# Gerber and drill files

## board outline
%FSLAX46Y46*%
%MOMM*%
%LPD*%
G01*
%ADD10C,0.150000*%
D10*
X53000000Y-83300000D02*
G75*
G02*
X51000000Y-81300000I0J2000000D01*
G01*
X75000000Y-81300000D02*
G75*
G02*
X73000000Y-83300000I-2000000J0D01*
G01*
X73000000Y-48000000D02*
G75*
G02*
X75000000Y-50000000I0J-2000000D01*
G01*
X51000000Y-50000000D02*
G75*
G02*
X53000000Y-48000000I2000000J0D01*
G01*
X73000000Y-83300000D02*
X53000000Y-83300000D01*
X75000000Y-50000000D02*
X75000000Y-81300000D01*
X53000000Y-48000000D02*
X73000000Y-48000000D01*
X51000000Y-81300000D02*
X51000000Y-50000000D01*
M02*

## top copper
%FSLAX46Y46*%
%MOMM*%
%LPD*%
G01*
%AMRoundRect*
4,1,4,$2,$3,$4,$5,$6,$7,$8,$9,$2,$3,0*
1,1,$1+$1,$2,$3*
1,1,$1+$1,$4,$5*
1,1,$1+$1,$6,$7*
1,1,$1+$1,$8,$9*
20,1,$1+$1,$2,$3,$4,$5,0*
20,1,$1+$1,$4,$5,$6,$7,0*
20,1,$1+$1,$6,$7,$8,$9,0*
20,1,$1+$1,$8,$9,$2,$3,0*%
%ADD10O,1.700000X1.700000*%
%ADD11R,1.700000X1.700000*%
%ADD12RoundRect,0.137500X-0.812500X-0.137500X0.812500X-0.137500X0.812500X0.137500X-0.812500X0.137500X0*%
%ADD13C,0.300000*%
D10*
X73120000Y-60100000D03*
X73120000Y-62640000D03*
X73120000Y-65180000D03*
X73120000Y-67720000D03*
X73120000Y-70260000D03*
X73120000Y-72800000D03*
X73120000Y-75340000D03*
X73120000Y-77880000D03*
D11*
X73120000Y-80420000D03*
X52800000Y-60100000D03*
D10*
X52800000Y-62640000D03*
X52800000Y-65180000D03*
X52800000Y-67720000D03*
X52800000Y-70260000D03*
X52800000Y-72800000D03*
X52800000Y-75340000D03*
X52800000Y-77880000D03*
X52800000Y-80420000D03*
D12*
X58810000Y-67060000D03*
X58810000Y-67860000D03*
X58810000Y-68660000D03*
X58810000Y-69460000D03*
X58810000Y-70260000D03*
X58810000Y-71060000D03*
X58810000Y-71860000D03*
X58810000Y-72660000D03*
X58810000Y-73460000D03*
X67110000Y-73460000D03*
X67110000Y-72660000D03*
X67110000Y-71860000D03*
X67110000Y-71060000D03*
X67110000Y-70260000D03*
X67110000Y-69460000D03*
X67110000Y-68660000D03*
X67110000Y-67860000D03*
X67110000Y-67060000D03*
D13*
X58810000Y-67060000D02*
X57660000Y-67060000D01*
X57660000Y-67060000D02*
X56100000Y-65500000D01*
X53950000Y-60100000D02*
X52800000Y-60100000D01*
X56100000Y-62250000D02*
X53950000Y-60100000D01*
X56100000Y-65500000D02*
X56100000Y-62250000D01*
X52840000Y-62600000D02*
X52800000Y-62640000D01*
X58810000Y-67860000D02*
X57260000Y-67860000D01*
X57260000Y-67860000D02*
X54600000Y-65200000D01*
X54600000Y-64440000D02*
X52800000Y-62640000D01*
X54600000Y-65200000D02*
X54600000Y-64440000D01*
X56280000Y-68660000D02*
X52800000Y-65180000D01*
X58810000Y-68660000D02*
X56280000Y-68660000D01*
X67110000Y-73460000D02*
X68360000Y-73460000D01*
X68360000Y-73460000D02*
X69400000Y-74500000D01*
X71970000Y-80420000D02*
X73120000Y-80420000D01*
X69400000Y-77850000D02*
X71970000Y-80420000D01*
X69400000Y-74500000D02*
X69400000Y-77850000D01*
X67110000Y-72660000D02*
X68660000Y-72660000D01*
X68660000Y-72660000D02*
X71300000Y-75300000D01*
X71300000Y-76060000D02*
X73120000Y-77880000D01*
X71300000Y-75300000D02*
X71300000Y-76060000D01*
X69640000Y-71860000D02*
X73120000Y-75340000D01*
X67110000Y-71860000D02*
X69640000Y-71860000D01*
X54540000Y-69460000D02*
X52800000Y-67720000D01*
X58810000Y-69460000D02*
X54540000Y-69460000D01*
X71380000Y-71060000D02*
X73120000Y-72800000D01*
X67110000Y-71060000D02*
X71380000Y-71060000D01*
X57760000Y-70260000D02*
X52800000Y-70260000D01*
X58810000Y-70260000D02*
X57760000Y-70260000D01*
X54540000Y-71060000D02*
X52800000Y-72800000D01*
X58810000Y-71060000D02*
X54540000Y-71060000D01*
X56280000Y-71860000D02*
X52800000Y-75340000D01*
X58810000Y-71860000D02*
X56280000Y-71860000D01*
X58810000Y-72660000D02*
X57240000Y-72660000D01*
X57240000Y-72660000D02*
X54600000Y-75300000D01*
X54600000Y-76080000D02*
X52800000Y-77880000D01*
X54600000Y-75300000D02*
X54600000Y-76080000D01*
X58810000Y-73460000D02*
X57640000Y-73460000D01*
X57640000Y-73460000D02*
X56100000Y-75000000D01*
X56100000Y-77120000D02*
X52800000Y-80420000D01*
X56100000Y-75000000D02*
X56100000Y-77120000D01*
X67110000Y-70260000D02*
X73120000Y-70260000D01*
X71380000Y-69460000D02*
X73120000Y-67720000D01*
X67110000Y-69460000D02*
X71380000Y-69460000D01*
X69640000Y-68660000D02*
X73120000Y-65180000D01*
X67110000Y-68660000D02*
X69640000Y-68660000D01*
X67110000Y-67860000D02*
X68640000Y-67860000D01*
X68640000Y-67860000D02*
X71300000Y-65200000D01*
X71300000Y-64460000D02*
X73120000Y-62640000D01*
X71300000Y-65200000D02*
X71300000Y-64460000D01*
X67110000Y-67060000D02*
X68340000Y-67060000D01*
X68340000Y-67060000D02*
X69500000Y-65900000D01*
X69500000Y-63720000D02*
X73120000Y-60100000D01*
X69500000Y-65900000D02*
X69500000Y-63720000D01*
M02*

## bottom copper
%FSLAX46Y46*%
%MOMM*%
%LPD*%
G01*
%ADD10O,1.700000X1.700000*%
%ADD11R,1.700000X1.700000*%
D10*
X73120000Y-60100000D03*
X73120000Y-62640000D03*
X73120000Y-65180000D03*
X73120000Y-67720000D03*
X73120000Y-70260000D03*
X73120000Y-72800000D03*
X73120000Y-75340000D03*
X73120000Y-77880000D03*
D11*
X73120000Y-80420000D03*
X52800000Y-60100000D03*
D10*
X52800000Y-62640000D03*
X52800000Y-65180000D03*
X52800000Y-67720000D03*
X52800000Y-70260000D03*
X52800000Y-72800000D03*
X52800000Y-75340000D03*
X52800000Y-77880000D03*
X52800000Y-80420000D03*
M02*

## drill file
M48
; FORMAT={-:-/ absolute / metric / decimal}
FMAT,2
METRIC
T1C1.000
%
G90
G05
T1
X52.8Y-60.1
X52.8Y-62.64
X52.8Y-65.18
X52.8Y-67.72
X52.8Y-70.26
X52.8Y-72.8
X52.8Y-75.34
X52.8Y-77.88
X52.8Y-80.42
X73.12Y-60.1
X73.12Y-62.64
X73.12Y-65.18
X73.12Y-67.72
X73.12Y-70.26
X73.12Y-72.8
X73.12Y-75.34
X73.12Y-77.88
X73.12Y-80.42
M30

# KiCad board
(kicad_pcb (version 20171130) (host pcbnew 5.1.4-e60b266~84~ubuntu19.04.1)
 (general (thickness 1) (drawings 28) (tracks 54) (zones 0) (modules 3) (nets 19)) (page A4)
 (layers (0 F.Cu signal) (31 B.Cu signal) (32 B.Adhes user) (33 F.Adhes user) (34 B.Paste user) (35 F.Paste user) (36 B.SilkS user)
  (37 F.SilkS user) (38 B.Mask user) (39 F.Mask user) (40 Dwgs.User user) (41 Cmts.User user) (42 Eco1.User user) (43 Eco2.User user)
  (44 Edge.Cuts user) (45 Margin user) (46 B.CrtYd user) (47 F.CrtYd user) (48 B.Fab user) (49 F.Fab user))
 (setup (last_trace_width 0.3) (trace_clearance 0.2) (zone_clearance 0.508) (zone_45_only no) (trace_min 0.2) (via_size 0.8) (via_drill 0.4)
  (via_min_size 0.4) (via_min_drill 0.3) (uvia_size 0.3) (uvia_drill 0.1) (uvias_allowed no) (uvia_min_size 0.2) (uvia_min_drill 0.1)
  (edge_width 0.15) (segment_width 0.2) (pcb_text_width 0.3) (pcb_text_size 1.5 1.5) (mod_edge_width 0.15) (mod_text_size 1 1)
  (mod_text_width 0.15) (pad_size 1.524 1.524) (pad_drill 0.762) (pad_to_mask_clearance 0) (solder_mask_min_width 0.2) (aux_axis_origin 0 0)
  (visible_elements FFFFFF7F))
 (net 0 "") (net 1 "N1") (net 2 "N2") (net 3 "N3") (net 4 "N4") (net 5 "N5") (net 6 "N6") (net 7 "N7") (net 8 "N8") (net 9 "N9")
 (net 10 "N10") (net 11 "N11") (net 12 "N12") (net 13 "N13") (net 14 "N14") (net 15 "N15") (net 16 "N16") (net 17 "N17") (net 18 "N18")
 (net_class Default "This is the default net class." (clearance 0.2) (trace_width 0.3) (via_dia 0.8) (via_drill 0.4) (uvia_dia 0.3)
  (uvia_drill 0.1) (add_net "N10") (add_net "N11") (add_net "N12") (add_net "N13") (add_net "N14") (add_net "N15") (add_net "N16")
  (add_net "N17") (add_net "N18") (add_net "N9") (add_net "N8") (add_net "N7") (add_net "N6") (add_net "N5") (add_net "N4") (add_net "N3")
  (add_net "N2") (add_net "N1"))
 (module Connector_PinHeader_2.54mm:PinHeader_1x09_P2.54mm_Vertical (layer F.Cu) (at 73.12 80.42 180)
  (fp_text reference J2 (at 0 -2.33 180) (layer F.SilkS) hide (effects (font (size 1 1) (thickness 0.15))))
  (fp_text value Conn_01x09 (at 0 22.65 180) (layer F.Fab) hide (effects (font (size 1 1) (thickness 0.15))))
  (pad 9 thru_hole oval (at 0 20.32 180) (size 1.7 1.7) (drill 1) (layers *.Cu *.Mask) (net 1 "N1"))
  (pad 8 thru_hole oval (at 0 17.78 180) (size 1.7 1.7) (drill 1) (layers *.Cu *.Mask) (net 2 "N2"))
  (pad 7 thru_hole oval (at 0 15.24 180) (size 1.7 1.7) (drill 1) (layers *.Cu *.Mask) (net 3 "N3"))
  (pad 6 thru_hole oval (at 0 12.7 180) (size 1.7 1.7) (drill 1) (layers *.Cu *.Mask) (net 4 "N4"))
  (pad 5 thru_hole oval (at 0 10.16 180) (size 1.7 1.7) (drill 1) (layers *.Cu *.Mask) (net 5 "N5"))
  (pad 4 thru_hole oval (at 0 7.62 180) (size 1.7 1.7) (drill 1) (layers *.Cu *.Mask) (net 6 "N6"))
  (pad 3 thru_hole oval (at 0 5.08 180) (size 1.7 1.7) (drill 1) (layers *.Cu *.Mask) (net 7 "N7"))
  (pad 2 thru_hole oval (at 0 2.54 180) (size 1.7 1.7) (drill 1) (layers *.Cu *.Mask) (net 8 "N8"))
  (pad 1 thru_hole rect (at 0 0 180) (size 1.7 1.7) (drill 1) (layers *.Cu *.Mask) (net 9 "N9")))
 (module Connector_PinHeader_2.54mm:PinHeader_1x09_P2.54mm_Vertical (layer F.Cu) (at 52.8 60.1)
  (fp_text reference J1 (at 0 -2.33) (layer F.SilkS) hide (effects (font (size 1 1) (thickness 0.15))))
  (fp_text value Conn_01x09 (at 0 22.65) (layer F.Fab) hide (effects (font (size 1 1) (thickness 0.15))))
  (pad 1 thru_hole rect (at 0 0) (size 1.7 1.7) (drill 1) (layers *.Cu *.Mask) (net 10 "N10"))
  (pad 2 thru_hole oval (at 0 2.54) (size 1.7 1.7) (drill 1) (layers *.Cu *.Mask) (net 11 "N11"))
  (pad 3 thru_hole oval (at 0 5.08) (size 1.7 1.7) (drill 1) (layers *.Cu *.Mask) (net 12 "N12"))
  (pad 4 thru_hole oval (at 0 7.62) (size 1.7 1.7) (drill 1) (layers *.Cu *.Mask) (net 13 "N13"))
  (pad 5 thru_hole oval (at 0 10.16) (size 1.7 1.7) (drill 1) (layers *.Cu *.Mask) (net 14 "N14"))
  (pad 6 thru_hole oval (at 0 12.7) (size 1.7 1.7) (drill 1) (layers *.Cu *.Mask) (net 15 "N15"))
  (pad 7 thru_hole oval (at 0 15.24) (size 1.7 1.7) (drill 1) (layers *.Cu *.Mask) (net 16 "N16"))
  (pad 8 thru_hole oval (at 0 17.78) (size 1.7 1.7) (drill 1) (layers *.Cu *.Mask) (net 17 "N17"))
  (pad 9 thru_hole oval (at 0 20.32) (size 1.7 1.7) (drill 1) (layers *.Cu *.Mask) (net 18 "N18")))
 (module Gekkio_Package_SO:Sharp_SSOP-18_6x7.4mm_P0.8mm (layer F.Cu) (at 62.96 70.26)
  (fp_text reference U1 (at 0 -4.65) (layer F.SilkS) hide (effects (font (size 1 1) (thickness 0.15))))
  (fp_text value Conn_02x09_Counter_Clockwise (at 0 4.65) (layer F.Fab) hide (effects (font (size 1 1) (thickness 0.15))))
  (pad 1 smd roundrect (at -4.15 -3.2) (size 1.9 0.55) (layers F.Cu F.Paste F.Mask) (roundrect_rratio 0.25) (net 10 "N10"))
  (pad 2 smd roundrect (at -4.15 -2.4) (size 1.9 0.55) (layers F.Cu F.Paste F.Mask) (roundrect_rratio 0.25) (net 11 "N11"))
  (pad 3 smd roundrect (at -4.15 -1.6) (size 1.9 0.55) (layers F.Cu F.Paste F.Mask) (roundrect_rratio 0.25) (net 12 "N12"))
  (pad 4 smd roundrect (at -4.15 -0.8) (size 1.9 0.55) (layers F.Cu F.Paste F.Mask) (roundrect_rratio 0.25) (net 13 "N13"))
  (pad 5 smd roundrect (at -4.15 0) (size 1.9 0.55) (layers F.Cu F.Paste F.Mask) (roundrect_rratio 0.25) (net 14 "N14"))
  (pad 6 smd roundrect (at -4.15 0.8) (size 1.9 0.55) (layers F.Cu F.Paste F.Mask) (roundrect_rratio 0.25) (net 15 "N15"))
  (pad 7 smd roundrect (at -4.15 1.6) (size 1.9 0.55) (layers F.Cu F.Paste F.Mask) (roundrect_rratio 0.25) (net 16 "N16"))
  (pad 8 smd roundrect (at -4.15 2.4) (size 1.9 0.55) (layers F.Cu F.Paste F.Mask) (roundrect_rratio 0.25) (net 17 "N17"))
  (pad 9 smd roundrect (at -4.15 3.2) (size 1.9 0.55) (layers F.Cu F.Paste F.Mask) (roundrect_rratio 0.25) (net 18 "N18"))
  (pad 10 smd roundrect (at 4.15 3.2) (size 1.9 0.55) (layers F.Cu F.Paste F.Mask) (roundrect_rratio 0.25) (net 9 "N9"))
  (pad 11 smd roundrect (at 4.15 2.4) (size 1.9 0.55) (layers F.Cu F.Paste F.Mask) (roundrect_rratio 0.25) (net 8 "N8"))
  (pad 12 smd roundrect (at 4.15 1.6) (size 1.9 0.55) (layers F.Cu F.Paste F.Mask) (roundrect_rratio 0.25) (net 7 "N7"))
  (pad 13 smd roundrect (at 4.15 0.8) (size 1.9 0.55) (layers F.Cu F.Paste F.Mask) (roundrect_rratio 0.25) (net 6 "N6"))
  (pad 14 smd roundrect (at 4.15 0) (size 1.9 0.55) (layers F.Cu F.Paste F.Mask) (roundrect_rratio 0.25) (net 5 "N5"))
  (pad 15 smd roundrect (at 4.15 -0.8) (size 1.9 0.55) (layers F.Cu F.Paste F.Mask) (roundrect_rratio 0.25) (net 4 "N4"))
  (pad 16 smd roundrect (at 4.15 -1.6) (size 1.9 0.55) (layers F.Cu F.Paste F.Mask) (roundrect_rratio 0.25) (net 3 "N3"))
  (pad 17 smd roundrect (at 4.15 -2.4) (size 1.9 0.55) (layers F.Cu F.Paste F.Mask) (roundrect_rratio 0.25) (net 2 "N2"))
  (pad 18 smd roundrect (at 4.15 -3.2) (size 1.9 0.55) (layers F.Cu F.Paste F.Mask) (roundrect_rratio 0.25) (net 1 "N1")))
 (gr_arc (start 53 81.3) (end 51 81.3) (angle -90) (layer Edge.Cuts) (width 0.15))
 (gr_arc (start 73 81.3) (end 73 83.3) (angle -90) (layer Edge.Cuts) (width 0.15))
 (gr_arc (start 73 50) (end 75 50) (angle -90) (layer Edge.Cuts) (width 0.15))
 (gr_arc (start 53 50) (end 53 48) (angle -90) (layer Edge.Cuts) (width 0.15))
 (gr_line (start 73 83.3) (end 53 83.3) (layer Edge.Cuts) (width 0.15))
 (gr_line (start 75 50) (end 75 81.3) (layer Edge.Cuts) (width 0.15))
 (gr_line (start 53 48) (end 73 48) (layer Edge.Cuts) (width 0.15))
 (gr_line (start 51 81.3) (end 51 50) (layer Edge.Cuts) (width 0.15))
 (segment (start 58.81 67.06) (end 57.66 67.06) (width 0.3) (layer F.Cu) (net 10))
 (segment (start 57.66 67.06) (end 56.1 65.5) (width 0.3) (layer F.Cu) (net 10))
 (segment (start 53.95 60.1) (end 52.8 60.1) (width 0.3) (layer F.Cu) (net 10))
 (segment (start 56.1 62.25) (end 53.95 60.1) (width 0.3) (layer F.Cu) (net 10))
 (segment (start 56.1 65.5) (end 56.1 62.25) (width 0.3) (layer F.Cu) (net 10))
 (segment (start 52.84 62.6) (end 52.8 62.64) (width 0.3) (layer F.Cu) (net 11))
 (segment (start 58.81 67.86) (end 57.26 67.86) (width 0.3) (layer F.Cu) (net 11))
 (segment (start 57.26 67.86) (end 54.6 65.2) (width 0.3) (layer F.Cu) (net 11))
 (segment (start 54.6 64.44) (end 52.8 62.64) (width 0.3) (layer F.Cu) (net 11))
 (segment (start 54.6 65.2) (end 54.6 64.44) (width 0.3) (layer F.Cu) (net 11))
 (segment (start 56.28 68.66) (end 52.8 65.18) (width 0.3) (layer F.Cu) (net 12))
 (segment (start 58.81 68.66) (end 56.28 68.66) (width 0.3) (layer F.Cu) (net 12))
 (segment (start 67.11 73.46) (end 68.36 73.46) (width 0.3) (layer F.Cu) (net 9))
 (segment (start 68.36 73.46) (end 69.4 74.5) (width 0.3) (layer F.Cu) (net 9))
 (segment (start 71.97 80.42) (end 73.12 80.42) (width 0.3) (layer F.Cu) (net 9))
 (segment (start 69.4 77.85) (end 71.97 80.42) (width 0.3) (layer F.Cu) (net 9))
 (segment (start 69.4 74.5) (end 69.4 77.85) (width 0.3) (layer F.Cu) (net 9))
 (segment (start 67.11 72.66) (end 68.66 72.66) (width 0.3) (layer F.Cu) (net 8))
 (segment (start 68.66 72.66) (end 71.3 75.3) (width 0.3) (layer F.Cu) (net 8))
 (segment (start 71.3 76.06) (end 73.12 77.88) (width 0.3) (layer F.Cu) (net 8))
 (segment (start 71.3 75.3) (end 71.3 76.06) (width 0.3) (layer F.Cu) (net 8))
 (segment (start 69.64 71.86) (end 73.12 75.34) (width 0.3) (layer F.Cu) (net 7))
 (segment (start 67.11 71.86) (end 69.64 71.86) (width 0.3) (layer F.Cu) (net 7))
 (segment (start 54.54 69.46) (end 52.8 67.72) (width 0.3) (layer F.Cu) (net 13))
 (segment (start 58.81 69.46) (end 54.54 69.46) (width 0.3) (layer F.Cu) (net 13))
 (segment (start 71.38 71.06) (end 73.12 72.8) (width 0.3) (layer F.Cu) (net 6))
 (segment (start 67.11 71.06) (end 71.38 71.06) (width 0.3) (layer F.Cu) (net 6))
 (segment (start 57.76 70.26) (end 52.8 70.26) (width 0.3) (layer F.Cu) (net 14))
 (segment (start 58.81 70.26) (end 57.76 70.26) (width 0.3) (layer F.Cu) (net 14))
 (segment (start 54.54 71.06) (end 52.8 72.8) (width 0.3) (layer F.Cu) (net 15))
 (segment (start 58.81 71.06) (end 54.54 71.06) (width 0.3) (layer F.Cu) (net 15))
 (segment (start 56.28 71.86) (end 52.8 75.34) (width 0.3) (layer F.Cu) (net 16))
 (segment (start 58.81 71.86) (end 56.28 71.86) (width 0.3) (layer F.Cu) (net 16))
 (segment (start 58.81 72.66) (end 57.24 72.66) (width 0.3) (layer F.Cu) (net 17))
 (segment (start 57.24 72.66) (end 54.6 75.3) (width 0.3) (layer F.Cu) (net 17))
 (segment (start 54.6 76.08) (end 52.8 77.88) (width 0.3) (layer F.Cu) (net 17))
 (segment (start 54.6 75.3) (end 54.6 76.08) (width 0.3) (layer F.Cu) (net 17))
 (segment (start 58.81 73.46) (end 57.64 73.46) (width 0.3) (layer F.Cu) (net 18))
 (segment (start 57.64 73.46) (end 56.1 75) (width 0.3) (layer F.Cu) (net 18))
 (segment (start 56.1 77.12) (end 52.8 80.42) (width 0.3) (layer F.Cu) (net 18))
 (segment (start 56.1 75) (end 56.1 77.12) (width 0.3) (layer F.Cu) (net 18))
 (segment (start 67.11 70.26) (end 73.12 70.26) (width 0.3) (layer F.Cu) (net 5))
 (segment (start 71.38 69.46) (end 73.12 67.72) (width 0.3) (layer F.Cu) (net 4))
 (segment (start 67.11 69.46) (end 71.38 69.46) (width 0.3) (layer F.Cu) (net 4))
 (segment (start 69.64 68.66) (end 73.12 65.18) (width 0.3) (layer F.Cu) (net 3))
 (segment (start 67.11 68.66) (end 69.64 68.66) (width 0.3) (layer F.Cu) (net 3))
 (segment (start 67.11 67.86) (end 68.64 67.86) (width 0.3) (layer F.Cu) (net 2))
 (segment (start 68.64 67.86) (end 71.3 65.2) (width 0.3) (layer F.Cu) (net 2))
 (segment (start 71.3 64.46) (end 73.12 62.64) (width 0.3) (layer F.Cu) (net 2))
 (segment (start 71.3 65.2) (end 71.3 64.46) (width 0.3) (layer F.Cu) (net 2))
 (segment (start 67.11 67.06) (end 68.34 67.06) (width 0.3) (layer F.Cu) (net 1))
 (segment (start 68.34 67.06) (end 69.5 65.9) (width 0.3) (layer F.Cu) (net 1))
 (segment (start 69.5 63.72) (end 73.12 60.1) (width 0.3) (layer F.Cu) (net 1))
 (segment (start 69.5 65.9) (end 69.5 63.72) (width 0.3) (layer F.Cu) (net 1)))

